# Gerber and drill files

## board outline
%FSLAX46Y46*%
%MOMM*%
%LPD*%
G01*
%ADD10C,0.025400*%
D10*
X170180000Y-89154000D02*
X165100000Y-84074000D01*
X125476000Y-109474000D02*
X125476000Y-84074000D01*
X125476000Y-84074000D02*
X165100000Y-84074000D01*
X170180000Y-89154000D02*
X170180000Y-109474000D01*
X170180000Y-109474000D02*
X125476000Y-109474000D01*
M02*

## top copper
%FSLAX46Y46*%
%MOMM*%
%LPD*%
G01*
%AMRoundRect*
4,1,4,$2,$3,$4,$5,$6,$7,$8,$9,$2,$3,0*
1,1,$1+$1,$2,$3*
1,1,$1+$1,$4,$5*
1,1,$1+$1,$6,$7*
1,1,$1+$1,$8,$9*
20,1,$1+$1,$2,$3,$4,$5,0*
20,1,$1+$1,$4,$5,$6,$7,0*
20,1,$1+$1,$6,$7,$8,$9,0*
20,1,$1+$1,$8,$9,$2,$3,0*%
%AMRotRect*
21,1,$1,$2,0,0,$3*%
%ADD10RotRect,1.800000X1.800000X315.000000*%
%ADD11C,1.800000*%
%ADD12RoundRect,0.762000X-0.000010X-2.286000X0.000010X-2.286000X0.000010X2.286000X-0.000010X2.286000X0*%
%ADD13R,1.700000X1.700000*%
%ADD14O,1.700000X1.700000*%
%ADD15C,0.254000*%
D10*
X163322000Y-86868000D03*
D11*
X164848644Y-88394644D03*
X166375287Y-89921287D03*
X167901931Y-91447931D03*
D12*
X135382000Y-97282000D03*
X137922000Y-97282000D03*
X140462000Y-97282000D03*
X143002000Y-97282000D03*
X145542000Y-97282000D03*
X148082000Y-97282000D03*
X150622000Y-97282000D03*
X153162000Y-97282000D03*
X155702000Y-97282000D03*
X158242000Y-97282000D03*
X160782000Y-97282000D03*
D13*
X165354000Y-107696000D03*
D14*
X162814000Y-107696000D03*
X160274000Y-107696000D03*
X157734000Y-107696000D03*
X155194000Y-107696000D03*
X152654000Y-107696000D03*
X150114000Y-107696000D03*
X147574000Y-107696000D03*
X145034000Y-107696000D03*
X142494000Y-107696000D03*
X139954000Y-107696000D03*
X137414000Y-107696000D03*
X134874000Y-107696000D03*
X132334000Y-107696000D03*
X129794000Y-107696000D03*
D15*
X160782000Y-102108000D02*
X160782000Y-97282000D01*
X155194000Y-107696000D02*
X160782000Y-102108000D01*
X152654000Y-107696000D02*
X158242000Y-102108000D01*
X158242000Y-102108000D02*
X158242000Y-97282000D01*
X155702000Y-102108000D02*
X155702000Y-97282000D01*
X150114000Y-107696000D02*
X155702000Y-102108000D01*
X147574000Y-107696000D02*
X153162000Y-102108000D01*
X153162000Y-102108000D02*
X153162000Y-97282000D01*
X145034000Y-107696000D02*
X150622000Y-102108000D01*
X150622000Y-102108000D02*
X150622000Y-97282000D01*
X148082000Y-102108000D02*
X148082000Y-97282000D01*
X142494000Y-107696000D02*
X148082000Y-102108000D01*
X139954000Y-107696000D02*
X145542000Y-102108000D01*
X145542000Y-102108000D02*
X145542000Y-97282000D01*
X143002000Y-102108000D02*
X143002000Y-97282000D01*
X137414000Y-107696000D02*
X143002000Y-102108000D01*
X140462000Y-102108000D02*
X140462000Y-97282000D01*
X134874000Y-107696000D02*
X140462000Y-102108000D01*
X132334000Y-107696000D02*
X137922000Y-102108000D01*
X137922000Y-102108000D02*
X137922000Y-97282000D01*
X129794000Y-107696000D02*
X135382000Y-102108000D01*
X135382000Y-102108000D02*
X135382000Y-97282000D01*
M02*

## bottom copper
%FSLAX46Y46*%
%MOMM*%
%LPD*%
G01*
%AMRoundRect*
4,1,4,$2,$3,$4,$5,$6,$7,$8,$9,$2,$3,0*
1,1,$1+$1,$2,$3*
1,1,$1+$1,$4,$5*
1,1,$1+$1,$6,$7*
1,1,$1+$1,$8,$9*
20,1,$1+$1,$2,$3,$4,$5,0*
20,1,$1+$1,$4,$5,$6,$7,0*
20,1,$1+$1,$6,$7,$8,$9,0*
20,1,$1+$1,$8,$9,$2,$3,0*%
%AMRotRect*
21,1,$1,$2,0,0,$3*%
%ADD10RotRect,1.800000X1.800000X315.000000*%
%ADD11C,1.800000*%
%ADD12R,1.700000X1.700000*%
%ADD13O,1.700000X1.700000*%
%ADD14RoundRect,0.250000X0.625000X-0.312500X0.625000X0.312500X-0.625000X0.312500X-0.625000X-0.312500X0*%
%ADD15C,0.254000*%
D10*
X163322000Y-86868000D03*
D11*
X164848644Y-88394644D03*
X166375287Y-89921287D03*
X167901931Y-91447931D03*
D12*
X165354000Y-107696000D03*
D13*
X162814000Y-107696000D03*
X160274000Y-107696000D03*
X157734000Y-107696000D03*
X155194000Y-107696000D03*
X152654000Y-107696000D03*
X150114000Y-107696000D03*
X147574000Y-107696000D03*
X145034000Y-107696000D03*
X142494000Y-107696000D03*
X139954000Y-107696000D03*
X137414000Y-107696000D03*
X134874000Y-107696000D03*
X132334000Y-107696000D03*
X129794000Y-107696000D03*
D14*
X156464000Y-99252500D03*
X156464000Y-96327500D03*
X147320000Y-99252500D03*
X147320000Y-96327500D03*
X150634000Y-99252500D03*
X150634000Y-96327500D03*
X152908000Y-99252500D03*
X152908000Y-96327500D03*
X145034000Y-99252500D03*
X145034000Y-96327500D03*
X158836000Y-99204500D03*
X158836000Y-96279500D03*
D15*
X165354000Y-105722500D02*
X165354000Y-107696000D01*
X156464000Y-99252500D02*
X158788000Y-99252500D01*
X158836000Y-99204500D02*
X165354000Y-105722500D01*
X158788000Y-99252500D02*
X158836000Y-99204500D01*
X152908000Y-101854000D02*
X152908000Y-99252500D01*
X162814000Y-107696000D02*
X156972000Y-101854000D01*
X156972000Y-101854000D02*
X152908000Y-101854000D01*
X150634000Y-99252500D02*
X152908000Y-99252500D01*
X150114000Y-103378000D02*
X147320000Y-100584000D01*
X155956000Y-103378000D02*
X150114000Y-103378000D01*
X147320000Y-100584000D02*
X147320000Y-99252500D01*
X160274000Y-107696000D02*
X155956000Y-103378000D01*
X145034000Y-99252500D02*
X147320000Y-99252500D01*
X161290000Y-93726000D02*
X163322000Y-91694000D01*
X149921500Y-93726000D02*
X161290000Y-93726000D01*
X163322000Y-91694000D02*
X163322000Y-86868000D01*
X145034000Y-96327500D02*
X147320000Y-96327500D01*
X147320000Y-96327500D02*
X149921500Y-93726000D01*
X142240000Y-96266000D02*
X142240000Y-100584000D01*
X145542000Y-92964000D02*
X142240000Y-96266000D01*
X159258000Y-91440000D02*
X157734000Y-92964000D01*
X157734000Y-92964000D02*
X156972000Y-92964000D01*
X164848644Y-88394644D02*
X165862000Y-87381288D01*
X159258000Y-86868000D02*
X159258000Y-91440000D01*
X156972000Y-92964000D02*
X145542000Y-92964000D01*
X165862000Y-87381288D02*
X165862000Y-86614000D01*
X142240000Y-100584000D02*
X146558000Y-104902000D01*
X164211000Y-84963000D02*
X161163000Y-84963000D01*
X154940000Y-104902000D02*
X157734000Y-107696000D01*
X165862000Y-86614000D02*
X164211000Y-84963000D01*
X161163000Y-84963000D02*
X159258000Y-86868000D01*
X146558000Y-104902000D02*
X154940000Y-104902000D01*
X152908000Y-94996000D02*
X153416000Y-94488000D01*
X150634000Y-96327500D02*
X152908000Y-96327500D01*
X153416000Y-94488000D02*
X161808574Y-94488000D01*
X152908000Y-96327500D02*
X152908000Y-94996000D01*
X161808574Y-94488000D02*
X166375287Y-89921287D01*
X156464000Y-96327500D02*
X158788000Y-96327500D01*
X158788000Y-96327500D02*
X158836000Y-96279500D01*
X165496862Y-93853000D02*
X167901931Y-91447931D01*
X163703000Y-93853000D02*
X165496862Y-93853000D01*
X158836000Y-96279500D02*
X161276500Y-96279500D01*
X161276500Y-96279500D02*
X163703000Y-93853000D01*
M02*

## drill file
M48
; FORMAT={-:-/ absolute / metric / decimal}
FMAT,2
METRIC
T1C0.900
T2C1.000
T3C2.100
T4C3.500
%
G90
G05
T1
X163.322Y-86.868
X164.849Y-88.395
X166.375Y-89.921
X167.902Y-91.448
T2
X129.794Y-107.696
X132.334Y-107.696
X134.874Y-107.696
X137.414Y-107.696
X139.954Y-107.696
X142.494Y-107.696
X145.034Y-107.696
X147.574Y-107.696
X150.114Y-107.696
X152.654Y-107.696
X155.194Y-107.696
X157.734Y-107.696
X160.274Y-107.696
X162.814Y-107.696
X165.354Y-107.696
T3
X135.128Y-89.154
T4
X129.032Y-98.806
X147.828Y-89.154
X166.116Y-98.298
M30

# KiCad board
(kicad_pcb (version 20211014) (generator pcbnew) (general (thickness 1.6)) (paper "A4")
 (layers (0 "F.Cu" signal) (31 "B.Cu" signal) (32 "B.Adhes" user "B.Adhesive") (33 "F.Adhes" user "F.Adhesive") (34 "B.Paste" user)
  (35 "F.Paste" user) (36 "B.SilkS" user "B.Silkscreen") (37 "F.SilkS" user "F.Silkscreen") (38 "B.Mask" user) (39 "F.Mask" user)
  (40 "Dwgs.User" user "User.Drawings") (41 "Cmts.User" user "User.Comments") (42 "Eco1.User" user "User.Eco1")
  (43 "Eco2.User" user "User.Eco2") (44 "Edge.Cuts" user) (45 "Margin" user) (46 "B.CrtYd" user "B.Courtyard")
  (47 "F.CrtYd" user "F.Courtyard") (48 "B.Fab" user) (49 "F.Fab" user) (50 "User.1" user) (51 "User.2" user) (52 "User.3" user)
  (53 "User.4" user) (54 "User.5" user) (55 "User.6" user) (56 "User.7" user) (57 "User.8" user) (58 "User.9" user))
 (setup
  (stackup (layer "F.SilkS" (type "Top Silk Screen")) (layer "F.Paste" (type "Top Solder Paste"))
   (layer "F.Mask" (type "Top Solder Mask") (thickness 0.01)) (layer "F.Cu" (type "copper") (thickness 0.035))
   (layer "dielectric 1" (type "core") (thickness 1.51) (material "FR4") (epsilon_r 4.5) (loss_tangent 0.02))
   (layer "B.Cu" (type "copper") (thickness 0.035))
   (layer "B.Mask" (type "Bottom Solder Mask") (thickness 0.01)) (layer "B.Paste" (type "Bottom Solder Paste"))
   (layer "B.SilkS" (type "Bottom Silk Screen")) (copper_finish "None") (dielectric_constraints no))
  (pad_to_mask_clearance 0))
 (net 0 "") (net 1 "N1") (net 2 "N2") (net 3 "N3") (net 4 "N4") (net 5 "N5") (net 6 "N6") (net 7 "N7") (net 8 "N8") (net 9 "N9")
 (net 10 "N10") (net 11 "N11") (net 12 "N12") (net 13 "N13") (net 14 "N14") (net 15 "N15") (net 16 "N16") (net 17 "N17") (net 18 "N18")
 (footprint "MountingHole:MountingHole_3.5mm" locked (layer "F.Cu") (at 147.828 89.154)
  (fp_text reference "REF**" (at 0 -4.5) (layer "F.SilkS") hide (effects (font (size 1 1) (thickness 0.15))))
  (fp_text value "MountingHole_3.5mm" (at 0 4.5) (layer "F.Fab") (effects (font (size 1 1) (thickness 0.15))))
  (pad "" np_thru_hole circle locked (at 0 0) (size 3.5 3.5) (drill 3.5) (layers *.Cu *.Mask)))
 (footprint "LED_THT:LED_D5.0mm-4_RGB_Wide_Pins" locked (layer "F.Cu") (at 163.322 86.868 -45)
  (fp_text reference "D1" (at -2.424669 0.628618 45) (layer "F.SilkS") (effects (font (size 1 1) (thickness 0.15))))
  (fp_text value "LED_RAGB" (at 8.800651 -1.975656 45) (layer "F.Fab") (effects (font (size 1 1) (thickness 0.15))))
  (pad "1" thru_hole rect locked (at 0 0 315) (size 1.8 1.8) (drill 0.9) (layers *.Cu *.Mask) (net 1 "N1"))
  (pad "2" thru_hole circle locked (at 2.159 0 315) (size 1.8 1.8) (drill 0.9) (layers *.Cu *.Mask) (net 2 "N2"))
  (pad "3" thru_hole circle locked (at 4.318 0 315) (size 1.8 1.8) (drill 0.9) (layers *.Cu *.Mask) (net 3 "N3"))
  (pad "4" thru_hole circle locked (at 6.477 0 315) (size 1.8 1.8) (drill 0.9) (layers *.Cu *.Mask) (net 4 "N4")))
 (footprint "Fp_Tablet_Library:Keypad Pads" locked (layer "F.Cu") (at 148.082 97.282)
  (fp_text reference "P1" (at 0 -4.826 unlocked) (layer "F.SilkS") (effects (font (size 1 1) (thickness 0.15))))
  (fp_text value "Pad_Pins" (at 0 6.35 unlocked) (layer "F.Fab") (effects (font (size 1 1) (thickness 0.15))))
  (pad "1" smd roundrect locked (at -12.7 0) (size 1.524 6.096) (layers "F.Cu" "F.Paste" "F.Mask") (roundrect_rratio 0.5) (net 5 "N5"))
  (pad "2" smd roundrect locked (at -10.16 0) (size 1.524 6.096) (layers "F.Cu" "F.Paste" "F.Mask") (roundrect_rratio 0.5) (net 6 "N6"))
  (pad "3" smd roundrect locked (at -7.62 0) (size 1.524 6.096) (layers "F.Cu" "F.Paste" "F.Mask") (roundrect_rratio 0.5) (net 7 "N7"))
  (pad "4" smd roundrect locked (at -5.08 0) (size 1.524 6.096) (layers "F.Cu" "F.Paste" "F.Mask") (roundrect_rratio 0.5) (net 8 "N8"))
  (pad "5" smd roundrect locked (at -2.54 0) (size 1.524 6.096) (layers "F.Cu" "F.Paste" "F.Mask") (roundrect_rratio 0.5) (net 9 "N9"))
  (pad "6" smd roundrect locked (at 0 0) (size 1.524 6.096) (layers "F.Cu" "F.Paste" "F.Mask") (roundrect_rratio 0.5) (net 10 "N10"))
  (pad "7" smd roundrect locked (at 2.54 0) (size 1.524 6.096) (layers "F.Cu" "F.Paste" "F.Mask") (roundrect_rratio 0.5) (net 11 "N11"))
  (pad "8" smd roundrect locked (at 5.08 0) (size 1.524 6.096) (layers "F.Cu" "F.Paste" "F.Mask") (roundrect_rratio 0.5) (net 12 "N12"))
  (pad "9" smd roundrect locked (at 7.62 0) (size 1.524 6.096) (layers "F.Cu" "F.Paste" "F.Mask") (roundrect_rratio 0.5) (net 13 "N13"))
  (pad "10" smd roundrect locked (at 10.16 0) (size 1.524 6.096) (layers "F.Cu" "F.Paste" "F.Mask") (roundrect_rratio 0.5) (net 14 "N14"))
  (pad "11" smd roundrect locked (at 12.7 0) (size 1.524 6.096) (layers "F.Cu" "F.Paste" "F.Mask") (roundrect_rratio 0.5) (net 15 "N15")))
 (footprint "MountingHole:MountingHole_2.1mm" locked (layer "F.Cu") (at 135.128 89.154)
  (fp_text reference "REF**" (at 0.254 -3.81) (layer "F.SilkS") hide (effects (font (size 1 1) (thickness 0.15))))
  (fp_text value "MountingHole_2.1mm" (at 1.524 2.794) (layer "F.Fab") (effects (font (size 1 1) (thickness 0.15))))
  (pad "" np_thru_hole circle locked (at 0 0) (size 2.1 2.1) (drill 2.1) (layers *.Cu *.Mask)))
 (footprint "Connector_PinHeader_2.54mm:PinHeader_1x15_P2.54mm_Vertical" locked (layer "F.Cu") (at 165.354 107.696 -90)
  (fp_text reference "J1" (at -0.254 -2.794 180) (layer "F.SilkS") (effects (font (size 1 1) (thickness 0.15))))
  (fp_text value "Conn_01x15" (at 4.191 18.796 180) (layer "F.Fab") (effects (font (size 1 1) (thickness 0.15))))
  (pad "1" thru_hole rect locked (at 0 0 270) (size 1.7 1.7) (drill 1) (layers *.Cu *.Mask) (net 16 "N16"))
  (pad "2" thru_hole oval locked (at 0 2.54 270) (size 1.7 1.7) (drill 1) (layers *.Cu *.Mask) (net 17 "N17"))
  (pad "3" thru_hole oval locked (at 0 5.08 270) (size 1.7 1.7) (drill 1) (layers *.Cu *.Mask) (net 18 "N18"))
  (pad "4" thru_hole oval locked (at 0 7.62 270) (size 1.7 1.7) (drill 1) (layers *.Cu *.Mask) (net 2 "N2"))
  (pad "5" thru_hole oval locked (at 0 10.16 270) (size 1.7 1.7) (drill 1) (layers *.Cu *.Mask) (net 15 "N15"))
  (pad "6" thru_hole oval locked (at 0 12.7 270) (size 1.7 1.7) (drill 1) (layers *.Cu *.Mask) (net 14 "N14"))
  (pad "7" thru_hole oval locked (at 0 15.24 270) (size 1.7 1.7) (drill 1) (layers *.Cu *.Mask) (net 13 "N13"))
  (pad "8" thru_hole oval locked (at 0 17.78 270) (size 1.7 1.7) (drill 1) (layers *.Cu *.Mask) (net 12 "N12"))
  (pad "9" thru_hole oval locked (at 0 20.32 270) (size 1.7 1.7) (drill 1) (layers *.Cu *.Mask) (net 11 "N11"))
  (pad "10" thru_hole oval locked (at 0 22.86 270) (size 1.7 1.7) (drill 1) (layers *.Cu *.Mask) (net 10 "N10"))
  (pad "11" thru_hole oval locked (at 0 25.4 270) (size 1.7 1.7) (drill 1) (layers *.Cu *.Mask) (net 9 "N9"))
  (pad "12" thru_hole oval locked (at 0 27.94 270) (size 1.7 1.7) (drill 1) (layers *.Cu *.Mask) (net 8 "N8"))
  (pad "13" thru_hole oval locked (at 0 30.48 270) (size 1.7 1.7) (drill 1) (layers *.Cu *.Mask) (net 7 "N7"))
  (pad "14" thru_hole oval locked (at 0 33.02 270) (size 1.7 1.7) (drill 1) (layers *.Cu *.Mask) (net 6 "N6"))
  (pad "15" thru_hole oval locked (at 0 35.56 270) (size 1.7 1.7) (drill 1) (layers *.Cu *.Mask) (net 5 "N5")))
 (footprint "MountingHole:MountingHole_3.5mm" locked (layer "F.Cu") (at 129.032 98.806)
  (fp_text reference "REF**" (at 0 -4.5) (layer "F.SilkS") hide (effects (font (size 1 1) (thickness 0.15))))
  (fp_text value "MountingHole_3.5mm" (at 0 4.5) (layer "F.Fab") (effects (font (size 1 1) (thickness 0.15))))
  (pad "" np_thru_hole circle locked (at 0 0) (size 3.5 3.5) (drill 3.5) (layers *.Cu *.Mask)))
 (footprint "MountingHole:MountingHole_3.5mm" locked (layer "F.Cu") (at 166.116 98.298)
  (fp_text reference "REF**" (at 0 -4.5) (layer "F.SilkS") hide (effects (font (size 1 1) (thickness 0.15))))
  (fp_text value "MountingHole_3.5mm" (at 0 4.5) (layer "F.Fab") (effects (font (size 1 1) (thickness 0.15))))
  (pad "" np_thru_hole circle locked (at 0 0) (size 3.5 3.5) (drill 3.5) (layers *.Cu *.Mask)))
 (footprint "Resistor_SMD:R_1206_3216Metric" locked (layer "B.Cu") (at 156.464 97.79 90)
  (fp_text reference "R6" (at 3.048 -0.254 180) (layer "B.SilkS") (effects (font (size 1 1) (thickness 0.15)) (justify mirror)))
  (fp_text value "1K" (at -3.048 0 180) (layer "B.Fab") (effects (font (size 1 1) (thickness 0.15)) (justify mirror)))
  (pad "1" smd roundrect locked (at -1.4625 0 90) (size 1.125 1.75) (layers "B.Cu" "B.Paste" "B.Mask") (roundrect_rratio 0.2222222222)
   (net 16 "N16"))
  (pad "2" smd roundrect locked (at 1.4625 0 90) (size 1.125 1.75) (layers "B.Cu" "B.Paste" "B.Mask") (roundrect_rratio 0.2222222222)
   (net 4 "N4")))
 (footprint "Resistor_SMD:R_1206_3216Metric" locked (layer "B.Cu") (at 147.32 97.79 90)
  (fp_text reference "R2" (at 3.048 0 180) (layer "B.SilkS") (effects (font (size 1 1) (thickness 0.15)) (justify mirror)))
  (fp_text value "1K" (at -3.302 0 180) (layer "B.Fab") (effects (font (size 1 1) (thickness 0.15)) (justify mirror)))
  (pad "1" smd roundrect locked (at -1.4625 0 90) (size 1.125 1.75) (layers "B.Cu" "B.Paste" "B.Mask") (roundrect_rratio 0.2222222222)
   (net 18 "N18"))
  (pad "2" smd roundrect locked (at 1.4625 0 90) (size 1.125 1.75) (layers "B.Cu" "B.Paste" "B.Mask") (roundrect_rratio 0.2222222222)
   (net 1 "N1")))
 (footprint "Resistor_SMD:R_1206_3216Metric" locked (layer "B.Cu") (at 150.634 97.79 90)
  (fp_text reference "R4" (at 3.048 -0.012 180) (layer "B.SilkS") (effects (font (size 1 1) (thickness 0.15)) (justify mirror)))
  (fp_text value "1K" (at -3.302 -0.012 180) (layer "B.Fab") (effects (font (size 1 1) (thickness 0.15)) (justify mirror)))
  (pad "1" smd roundrect locked (at -1.4625 0 90) (size 1.125 1.75) (layers "B.Cu" "B.Paste" "B.Mask") (roundrect_rratio 0.2222222222)
   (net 17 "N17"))
  (pad "2" smd roundrect locked (at 1.4625 0 90) (size 1.125 1.75) (layers "B.Cu" "B.Paste" "B.Mask") (roundrect_rratio 0.2222222222)
   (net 3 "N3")))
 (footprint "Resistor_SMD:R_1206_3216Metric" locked (layer "B.Cu") (at 152.908 97.79 90)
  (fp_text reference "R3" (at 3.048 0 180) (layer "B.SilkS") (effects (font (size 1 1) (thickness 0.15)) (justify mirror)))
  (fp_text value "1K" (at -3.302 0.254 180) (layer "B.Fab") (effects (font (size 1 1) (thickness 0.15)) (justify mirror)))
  (pad "1" smd roundrect locked (at -1.4625 0 90) (size 1.125 1.75) (layers "B.Cu" "B.Paste" "B.Mask") (roundrect_rratio 0.2222222222)
   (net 17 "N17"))
  (pad "2" smd roundrect locked (at 1.4625 0 90) (size 1.125 1.75) (layers "B.Cu" "B.Paste" "B.Mask") (roundrect_rratio 0.2222222222)
   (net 3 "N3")))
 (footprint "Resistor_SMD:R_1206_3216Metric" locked (layer "B.Cu") (at 145.034 97.79 90)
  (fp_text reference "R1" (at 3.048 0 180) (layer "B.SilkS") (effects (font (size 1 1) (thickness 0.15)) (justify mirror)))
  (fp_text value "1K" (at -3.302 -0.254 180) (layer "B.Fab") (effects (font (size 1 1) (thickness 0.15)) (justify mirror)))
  (pad "1" smd roundrect locked (at -1.4625 0 90) (size 1.125 1.75) (layers "B.Cu" "B.Paste" "B.Mask") (roundrect_rratio 0.2222222222)
   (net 18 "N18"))
  (pad "2" smd roundrect locked (at 1.4625 0 90) (size 1.125 1.75) (layers "B.Cu" "B.Paste" "B.Mask") (roundrect_rratio 0.2222222222)
   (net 1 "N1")))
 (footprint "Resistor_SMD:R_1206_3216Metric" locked (layer "B.Cu") (at 158.836 97.742 90)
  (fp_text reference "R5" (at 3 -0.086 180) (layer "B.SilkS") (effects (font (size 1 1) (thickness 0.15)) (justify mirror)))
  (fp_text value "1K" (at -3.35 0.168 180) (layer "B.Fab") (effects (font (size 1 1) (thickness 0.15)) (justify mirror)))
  (pad "1" smd roundrect locked (at -1.4625 0 90) (size 1.125 1.75) (layers "B.Cu" "B.Paste" "B.Mask") (roundrect_rratio 0.2222222222)
   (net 16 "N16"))
  (pad "2" smd roundrect locked (at 1.4625 0 90) (size 1.125 1.75) (layers "B.Cu" "B.Paste" "B.Mask") (roundrect_rratio 0.2222222222)
   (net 4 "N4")))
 (gr_line (start 170.18 89.154) (end 165.1 84.074) (layer "Edge.Cuts") (width 0.0254))
 (gr_line (start 125.476 109.474) (end 125.476 84.074) (layer "Edge.Cuts") (width 0.0254))
 (gr_line (start 125.476 84.074) (end 165.1 84.074) (layer "Edge.Cuts") (width 0.0254))
 (gr_line (start 170.18 89.154) (end 170.18 109.474) (layer "Edge.Cuts") (width 0.0254))
 (gr_line (start 170.18 109.474) (end 125.476 109.474) (layer "Edge.Cuts") (width 0.0254))
 (segment (start 165.354 105.7225) (end 165.354 107.696) (width 0.254) (layer "B.Cu") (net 16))
 (segment (start 156.464 99.2525) (end 158.788 99.2525) (width 0.254) (layer "B.Cu") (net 16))
 (segment (start 158.836 99.2045) (end 165.354 105.7225) (width 0.254) (layer "B.Cu") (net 16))
 (segment (start 158.788 99.2525) (end 158.836 99.2045) (width 0.254) (layer "B.Cu") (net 16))
 (segment (start 152.908 101.854) (end 152.908 99.2525) (width 0.254) (layer "B.Cu") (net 17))
 (segment (start 162.814 107.696) (end 156.972 101.854) (width 0.254) (layer "B.Cu") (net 17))
 (segment (start 156.972 101.854) (end 152.908 101.854) (width 0.254) (layer "B.Cu") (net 17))
 (segment (start 150.634 99.2525) (end 152.908 99.2525) (width 0.254) (layer "B.Cu") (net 17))
 (segment (start 150.114 103.378) (end 147.32 100.584) (width 0.254) (layer "B.Cu") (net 18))
 (segment (start 155.956 103.378) (end 150.114 103.378) (width 0.254) (layer "B.Cu") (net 18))
 (segment (start 147.32 100.584) (end 147.32 99.2525) (width 0.254) (layer "B.Cu") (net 18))
 (segment (start 160.274 107.696) (end 155.956 103.378) (width 0.254) (layer "B.Cu") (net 18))
 (segment (start 145.034 99.2525) (end 147.32 99.2525) (width 0.254) (layer "B.Cu") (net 18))
 (segment (start 160.782 102.108) (end 160.782 97.282) (width 0.254) (layer "F.Cu") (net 15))
 (segment (start 155.194 107.696) (end 160.782 102.108) (width 0.254) (layer "F.Cu") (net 15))
 (segment (start 152.654 107.696) (end 158.242 102.108) (width 0.254) (layer "F.Cu") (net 14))
 (segment (start 158.242 102.108) (end 158.242 97.282) (width 0.254) (layer "F.Cu") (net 14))
 (segment (start 155.702 102.108) (end 155.702 97.282) (width 0.254) (layer "F.Cu") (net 13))
 (segment (start 150.114 107.696) (end 155.702 102.108) (width 0.254) (layer "F.Cu") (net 13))
 (segment (start 147.574 107.696) (end 153.162 102.108) (width 0.254) (layer "F.Cu") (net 12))
 (segment (start 153.162 102.108) (end 153.162 97.282) (width 0.254) (layer "F.Cu") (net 12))
 (segment (start 145.034 107.696) (end 150.622 102.108) (width 0.254) (layer "F.Cu") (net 11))
 (segment (start 150.622 102.108) (end 150.622 97.282) (width 0.254) (layer "F.Cu") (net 11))
 (segment (start 148.082 102.108) (end 148.082 97.282) (width 0.254) (layer "F.Cu") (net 10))
 (segment (start 142.494 107.696) (end 148.082 102.108) (width 0.254) (layer "F.Cu") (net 10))
 (segment (start 139.954 107.696) (end 145.542 102.108) (width 0.254) (layer "F.Cu") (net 9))
 (segment (start 145.542 102.108) (end 145.542 97.282) (width 0.254) (layer "F.Cu") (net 9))
 (segment (start 161.29 93.726) (end 163.322 91.694) (width 0.254) (layer "B.Cu") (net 1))
 (segment (start 149.9215 93.726) (end 161.29 93.726) (width 0.254) (layer "B.Cu") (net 1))
 (segment (start 163.322 91.694) (end 163.322 86.868) (width 0.254) (layer "B.Cu") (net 1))
 (segment (start 145.034 96.3275) (end 147.32 96.3275) (width 0.254) (layer "B.Cu") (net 1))
 (segment (start 147.32 96.3275) (end 149.9215 93.726) (width 0.254) (layer "B.Cu") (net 1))
 (segment (start 142.24 96.266) (end 142.24 100.584) (width 0.254) (layer "B.Cu") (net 2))
 (segment (start 145.542 92.964) (end 142.24 96.266) (width 0.254) (layer "B.Cu") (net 2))
 (segment (start 159.258 91.44) (end 157.734 92.964) (width 0.254) (layer "B.Cu") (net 2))
 (segment (start 157.734 92.964) (end 156.972 92.964) (width 0.254) (layer "B.Cu") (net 2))
 (segment (start 164.848644 88.394644) (end 165.862 87.381288) (width 0.254) (layer "B.Cu") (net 2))
 (segment (start 159.258 86.868) (end 159.258 91.44) (width 0.254) (layer "B.Cu") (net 2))
 (segment (start 156.972 92.964) (end 145.542 92.964) (width 0.254) (layer "B.Cu") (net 2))
 (segment (start 165.862 87.381288) (end 165.862 86.614) (width 0.254) (layer "B.Cu") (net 2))
 (segment (start 142.24 100.584) (end 146.558 104.902) (width 0.254) (layer "B.Cu") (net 2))
 (segment (start 164.211 84.963) (end 161.163 84.963) (width 0.254) (layer "B.Cu") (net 2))
 (segment (start 154.94 104.902) (end 157.734 107.696) (width 0.254) (layer "B.Cu") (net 2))
 (segment (start 165.862 86.614) (end 164.211 84.963) (width 0.254) (layer "B.Cu") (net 2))
 (segment (start 161.163 84.963) (end 159.258 86.868) (width 0.254) (layer "B.Cu") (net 2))
 (segment (start 146.558 104.902) (end 154.94 104.902) (width 0.254) (layer "B.Cu") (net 2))
 (segment (start 152.908 94.996) (end 153.416 94.488) (width 0.254) (layer "B.Cu") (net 3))
 (segment (start 150.634 96.3275) (end 152.908 96.3275) (width 0.254) (layer "B.Cu") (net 3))
 (segment (start 153.416 94.488) (end 161.808574 94.488) (width 0.254) (layer "B.Cu") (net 3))
 (segment (start 152.908 96.3275) (end 152.908 94.996) (width 0.254) (layer "B.Cu") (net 3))
 (segment (start 161.808574 94.488) (end 166.375287 89.921287) (width 0.254) (layer "B.Cu") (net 3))
 (segment (start 156.464 96.3275) (end 158.788 96.3275) (width 0.254) (layer "B.Cu") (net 4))
 (segment (start 158.788 96.3275) (end 158.836 96.2795) (width 0.254) (layer "B.Cu") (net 4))
 (segment (start 165.496862 93.853) (end 167.901931 91.447931) (width 0.254) (layer "B.Cu") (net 4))
 (segment (start 163.703 93.853) (end 165.496862 93.853) (width 0.254) (layer "B.Cu") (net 4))
 (segment (start 158.836 96.2795) (end 161.2765 96.2795) (width 0.254) (layer "B.Cu") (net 4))
 (segment (start 161.2765 96.2795) (end 163.703 93.853) (width 0.254) (layer "B.Cu") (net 4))
 (segment (start 143.002 102.108) (end 143.002 97.282) (width 0.254) (layer "F.Cu") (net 8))
 (segment (start 137.414 107.696) (end 143.002 102.108) (width 0.254) (layer "F.Cu") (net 8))
 (segment (start 140.462 102.108) (end 140.462 97.282) (width 0.254) (layer "F.Cu") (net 7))
 (segment (start 134.874 107.696) (end 140.462 102.108) (width 0.254) (layer "F.Cu") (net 7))
 (segment (start 132.334 107.696) (end 137.922 102.108) (width 0.254) (layer "F.Cu") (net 6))
 (segment (start 137.922 102.108) (end 137.922 97.282) (width 0.254) (layer "F.Cu") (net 6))
 (segment (start 129.794 107.696) (end 135.382 102.108) (width 0.254) (layer "F.Cu") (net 5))
 (segment (start 135.382 102.108) (end 135.382 97.282) (width 0.254) (layer "F.Cu") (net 5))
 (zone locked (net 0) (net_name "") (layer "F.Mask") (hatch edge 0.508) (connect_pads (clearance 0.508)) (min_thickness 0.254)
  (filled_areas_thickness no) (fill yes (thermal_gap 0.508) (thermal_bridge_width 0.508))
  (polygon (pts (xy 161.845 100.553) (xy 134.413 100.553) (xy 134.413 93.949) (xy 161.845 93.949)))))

